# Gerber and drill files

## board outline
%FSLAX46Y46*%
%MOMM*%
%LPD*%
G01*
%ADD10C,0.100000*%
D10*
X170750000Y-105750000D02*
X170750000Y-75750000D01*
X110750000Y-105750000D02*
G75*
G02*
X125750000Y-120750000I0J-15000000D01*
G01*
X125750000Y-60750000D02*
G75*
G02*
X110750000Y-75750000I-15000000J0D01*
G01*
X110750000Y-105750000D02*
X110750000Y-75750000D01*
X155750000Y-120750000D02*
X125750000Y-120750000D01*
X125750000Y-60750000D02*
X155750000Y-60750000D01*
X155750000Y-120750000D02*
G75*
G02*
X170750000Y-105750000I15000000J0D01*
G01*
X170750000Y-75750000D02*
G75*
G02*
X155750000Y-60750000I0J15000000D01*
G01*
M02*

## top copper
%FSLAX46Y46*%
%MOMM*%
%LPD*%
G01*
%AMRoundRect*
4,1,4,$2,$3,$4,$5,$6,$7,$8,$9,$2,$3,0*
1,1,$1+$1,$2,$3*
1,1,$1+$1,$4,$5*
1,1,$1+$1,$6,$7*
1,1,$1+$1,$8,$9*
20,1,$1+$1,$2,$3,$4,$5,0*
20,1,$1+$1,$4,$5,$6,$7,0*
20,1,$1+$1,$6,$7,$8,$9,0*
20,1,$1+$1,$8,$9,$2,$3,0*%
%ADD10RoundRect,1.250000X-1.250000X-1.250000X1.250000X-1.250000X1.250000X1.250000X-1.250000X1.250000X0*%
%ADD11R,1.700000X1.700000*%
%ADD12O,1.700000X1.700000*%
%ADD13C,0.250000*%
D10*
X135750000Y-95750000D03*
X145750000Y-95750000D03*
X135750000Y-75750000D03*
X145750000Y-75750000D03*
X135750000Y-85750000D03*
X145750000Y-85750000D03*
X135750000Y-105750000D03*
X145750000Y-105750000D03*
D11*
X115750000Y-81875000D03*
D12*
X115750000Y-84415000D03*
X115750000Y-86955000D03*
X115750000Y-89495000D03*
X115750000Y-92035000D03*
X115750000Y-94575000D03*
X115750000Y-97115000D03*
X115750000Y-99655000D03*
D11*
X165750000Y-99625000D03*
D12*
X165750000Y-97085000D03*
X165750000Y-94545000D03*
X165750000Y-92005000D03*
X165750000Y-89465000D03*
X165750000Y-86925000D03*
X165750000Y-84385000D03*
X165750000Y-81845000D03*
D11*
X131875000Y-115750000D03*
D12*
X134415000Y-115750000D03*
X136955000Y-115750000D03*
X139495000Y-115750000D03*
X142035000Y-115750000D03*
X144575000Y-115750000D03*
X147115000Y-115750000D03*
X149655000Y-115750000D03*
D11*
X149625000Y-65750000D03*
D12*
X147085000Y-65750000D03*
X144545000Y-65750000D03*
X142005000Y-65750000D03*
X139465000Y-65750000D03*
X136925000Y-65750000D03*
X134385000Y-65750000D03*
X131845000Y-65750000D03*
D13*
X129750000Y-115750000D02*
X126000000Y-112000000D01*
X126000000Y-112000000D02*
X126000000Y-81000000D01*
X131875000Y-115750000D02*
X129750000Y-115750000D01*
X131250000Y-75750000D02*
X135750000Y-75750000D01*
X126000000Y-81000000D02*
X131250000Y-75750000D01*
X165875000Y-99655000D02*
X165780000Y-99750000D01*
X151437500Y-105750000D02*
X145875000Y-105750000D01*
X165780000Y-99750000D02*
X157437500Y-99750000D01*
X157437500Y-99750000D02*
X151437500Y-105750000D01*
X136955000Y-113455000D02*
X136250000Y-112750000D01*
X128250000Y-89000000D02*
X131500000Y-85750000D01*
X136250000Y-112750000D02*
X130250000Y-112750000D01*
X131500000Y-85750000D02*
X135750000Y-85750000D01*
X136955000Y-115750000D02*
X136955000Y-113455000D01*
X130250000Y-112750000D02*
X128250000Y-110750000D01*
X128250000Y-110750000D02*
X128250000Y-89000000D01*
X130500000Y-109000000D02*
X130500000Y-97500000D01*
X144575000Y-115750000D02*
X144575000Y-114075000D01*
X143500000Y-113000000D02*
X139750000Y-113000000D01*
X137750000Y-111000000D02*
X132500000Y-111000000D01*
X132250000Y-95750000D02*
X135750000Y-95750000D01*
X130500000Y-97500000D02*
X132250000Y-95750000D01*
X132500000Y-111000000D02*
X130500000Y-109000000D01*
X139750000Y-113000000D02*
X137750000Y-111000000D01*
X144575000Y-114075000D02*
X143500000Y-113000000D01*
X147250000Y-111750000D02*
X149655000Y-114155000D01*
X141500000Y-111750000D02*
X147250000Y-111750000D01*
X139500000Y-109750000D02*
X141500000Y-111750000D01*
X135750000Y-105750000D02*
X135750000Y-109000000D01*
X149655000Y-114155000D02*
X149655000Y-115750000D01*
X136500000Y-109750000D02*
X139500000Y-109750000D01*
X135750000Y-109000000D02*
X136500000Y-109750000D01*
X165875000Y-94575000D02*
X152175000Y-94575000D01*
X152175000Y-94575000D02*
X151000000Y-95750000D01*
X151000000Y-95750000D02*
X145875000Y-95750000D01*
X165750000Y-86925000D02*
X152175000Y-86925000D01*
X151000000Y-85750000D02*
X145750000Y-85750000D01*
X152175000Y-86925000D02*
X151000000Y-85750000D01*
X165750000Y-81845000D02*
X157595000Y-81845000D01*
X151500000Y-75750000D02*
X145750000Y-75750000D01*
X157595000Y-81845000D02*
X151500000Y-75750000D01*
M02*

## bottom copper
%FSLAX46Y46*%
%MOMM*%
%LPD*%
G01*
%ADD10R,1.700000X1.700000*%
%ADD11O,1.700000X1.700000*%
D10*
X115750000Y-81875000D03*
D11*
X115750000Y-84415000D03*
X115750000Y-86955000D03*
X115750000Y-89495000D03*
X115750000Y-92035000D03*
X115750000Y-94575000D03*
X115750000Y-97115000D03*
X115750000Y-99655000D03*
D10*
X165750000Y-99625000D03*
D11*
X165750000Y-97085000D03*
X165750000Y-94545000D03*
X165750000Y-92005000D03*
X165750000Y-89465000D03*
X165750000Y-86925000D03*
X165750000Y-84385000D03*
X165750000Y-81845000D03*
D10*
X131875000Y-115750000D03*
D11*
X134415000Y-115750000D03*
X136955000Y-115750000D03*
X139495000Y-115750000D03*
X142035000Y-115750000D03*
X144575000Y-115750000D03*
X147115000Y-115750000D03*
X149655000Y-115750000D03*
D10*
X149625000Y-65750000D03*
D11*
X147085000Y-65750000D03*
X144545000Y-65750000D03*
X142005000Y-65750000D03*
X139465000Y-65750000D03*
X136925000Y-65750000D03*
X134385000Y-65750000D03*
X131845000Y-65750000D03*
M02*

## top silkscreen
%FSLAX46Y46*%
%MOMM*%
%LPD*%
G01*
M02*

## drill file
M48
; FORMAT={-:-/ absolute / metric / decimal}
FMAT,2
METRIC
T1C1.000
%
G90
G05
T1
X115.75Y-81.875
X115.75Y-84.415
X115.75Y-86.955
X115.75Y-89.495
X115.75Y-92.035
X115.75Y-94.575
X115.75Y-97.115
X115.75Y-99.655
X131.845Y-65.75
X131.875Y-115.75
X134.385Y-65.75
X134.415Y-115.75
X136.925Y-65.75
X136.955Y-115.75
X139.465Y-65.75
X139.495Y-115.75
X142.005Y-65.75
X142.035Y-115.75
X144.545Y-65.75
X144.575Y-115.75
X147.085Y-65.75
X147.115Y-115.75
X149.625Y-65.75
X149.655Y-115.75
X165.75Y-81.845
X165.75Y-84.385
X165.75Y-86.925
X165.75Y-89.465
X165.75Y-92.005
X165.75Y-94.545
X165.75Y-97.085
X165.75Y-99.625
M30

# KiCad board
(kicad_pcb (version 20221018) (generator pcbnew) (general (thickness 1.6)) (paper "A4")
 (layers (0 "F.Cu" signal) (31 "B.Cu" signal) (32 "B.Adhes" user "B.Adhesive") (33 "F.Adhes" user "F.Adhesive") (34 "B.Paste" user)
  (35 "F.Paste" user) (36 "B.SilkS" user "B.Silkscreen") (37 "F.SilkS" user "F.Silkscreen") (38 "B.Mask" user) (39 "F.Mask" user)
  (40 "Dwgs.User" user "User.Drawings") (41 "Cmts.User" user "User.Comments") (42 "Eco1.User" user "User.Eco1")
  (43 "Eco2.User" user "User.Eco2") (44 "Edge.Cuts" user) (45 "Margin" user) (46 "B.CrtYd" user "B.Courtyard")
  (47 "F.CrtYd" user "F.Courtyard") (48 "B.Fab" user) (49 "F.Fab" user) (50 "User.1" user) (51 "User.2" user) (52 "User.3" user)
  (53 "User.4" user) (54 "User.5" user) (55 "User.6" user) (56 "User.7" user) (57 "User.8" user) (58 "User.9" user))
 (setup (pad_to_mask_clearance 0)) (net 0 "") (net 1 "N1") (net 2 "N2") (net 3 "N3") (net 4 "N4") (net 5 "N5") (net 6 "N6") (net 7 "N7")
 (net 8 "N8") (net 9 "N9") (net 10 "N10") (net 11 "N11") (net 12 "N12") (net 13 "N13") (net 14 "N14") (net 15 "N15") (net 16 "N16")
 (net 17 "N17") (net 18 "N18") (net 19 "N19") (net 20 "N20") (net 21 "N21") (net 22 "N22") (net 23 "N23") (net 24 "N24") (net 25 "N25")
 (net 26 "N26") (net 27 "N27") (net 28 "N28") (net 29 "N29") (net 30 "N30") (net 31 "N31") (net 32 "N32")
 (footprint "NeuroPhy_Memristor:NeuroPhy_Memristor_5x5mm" (layer "F.Cu") (at 140.75 95.75)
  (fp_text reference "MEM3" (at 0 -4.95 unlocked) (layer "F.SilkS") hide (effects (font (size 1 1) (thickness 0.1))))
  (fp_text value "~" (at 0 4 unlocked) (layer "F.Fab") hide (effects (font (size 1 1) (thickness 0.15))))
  (pad "1" smd roundrect (at -5 0) (size 5 5) (layers "F.Cu" "F.Mask") (roundrect_rratio 0.25) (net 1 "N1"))
  (pad "2" smd roundrect (at 5 0) (size 5 5) (layers "F.Cu" "F.Mask") (roundrect_rratio 0.25) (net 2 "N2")))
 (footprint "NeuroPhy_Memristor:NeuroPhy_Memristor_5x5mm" (layer "F.Cu") (at 140.75 75.75)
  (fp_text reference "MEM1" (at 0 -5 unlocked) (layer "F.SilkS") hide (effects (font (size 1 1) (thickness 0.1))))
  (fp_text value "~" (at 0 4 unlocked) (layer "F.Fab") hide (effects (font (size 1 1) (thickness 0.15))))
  (pad "1" smd roundrect (at -5 0) (size 5 5) (layers "F.Cu" "F.Mask") (roundrect_rratio 0.25) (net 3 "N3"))
  (pad "2" smd roundrect (at 5 0) (size 5 5) (layers "F.Cu" "F.Mask") (roundrect_rratio 0.25) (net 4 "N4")))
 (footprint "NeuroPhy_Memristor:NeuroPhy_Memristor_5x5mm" (layer "F.Cu") (at 140.75 85.75)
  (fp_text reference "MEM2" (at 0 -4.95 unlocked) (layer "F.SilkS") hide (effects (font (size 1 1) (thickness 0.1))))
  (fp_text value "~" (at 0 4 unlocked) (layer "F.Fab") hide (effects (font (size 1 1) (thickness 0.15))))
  (pad "1" smd roundrect (at -5 0) (size 5 5) (layers "F.Cu" "F.Mask") (roundrect_rratio 0.25) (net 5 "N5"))
  (pad "2" smd roundrect (at 5 0) (size 5 5) (layers "F.Cu" "F.Mask") (roundrect_rratio 0.25) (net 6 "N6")))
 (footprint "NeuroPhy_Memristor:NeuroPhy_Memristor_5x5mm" (layer "F.Cu") (at 140.75 105.75)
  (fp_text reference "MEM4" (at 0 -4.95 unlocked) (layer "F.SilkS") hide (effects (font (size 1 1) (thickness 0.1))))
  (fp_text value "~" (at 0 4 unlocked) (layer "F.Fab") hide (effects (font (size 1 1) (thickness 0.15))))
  (pad "1" smd roundrect (at -5 0) (size 5 5) (layers "F.Cu" "F.Mask") (roundrect_rratio 0.25) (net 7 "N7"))
  (pad "2" smd roundrect (at 5 0) (size 5 5) (layers "F.Cu" "F.Mask") (roundrect_rratio 0.25) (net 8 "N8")))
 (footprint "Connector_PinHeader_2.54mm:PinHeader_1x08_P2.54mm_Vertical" (layer "B.Cu") (at 115.75 81.875 180)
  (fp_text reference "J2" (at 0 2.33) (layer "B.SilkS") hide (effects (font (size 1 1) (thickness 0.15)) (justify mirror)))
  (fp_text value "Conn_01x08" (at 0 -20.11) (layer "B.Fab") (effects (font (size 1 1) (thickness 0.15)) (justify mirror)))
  (pad "1" thru_hole rect (at 0 0 180) (size 1.7 1.7) (drill 1) (layers "*.Cu" "*.Mask") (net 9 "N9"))
  (pad "2" thru_hole oval (at 0 -2.54 180) (size 1.7 1.7) (drill 1) (layers "*.Cu" "*.Mask") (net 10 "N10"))
  (pad "3" thru_hole oval (at 0 -5.08 180) (size 1.7 1.7) (drill 1) (layers "*.Cu" "*.Mask") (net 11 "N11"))
  (pad "4" thru_hole oval (at 0 -7.62 180) (size 1.7 1.7) (drill 1) (layers "*.Cu" "*.Mask") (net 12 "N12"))
  (pad "5" thru_hole oval (at 0 -10.16 180) (size 1.7 1.7) (drill 1) (layers "*.Cu" "*.Mask") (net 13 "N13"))
  (pad "6" thru_hole oval (at 0 -12.7 180) (size 1.7 1.7) (drill 1) (layers "*.Cu" "*.Mask") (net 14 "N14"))
  (pad "7" thru_hole oval (at 0 -15.24 180) (size 1.7 1.7) (drill 1) (layers "*.Cu" "*.Mask") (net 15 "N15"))
  (pad "8" thru_hole oval (at 0 -17.78 180) (size 1.7 1.7) (drill 1) (layers "*.Cu" "*.Mask") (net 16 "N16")))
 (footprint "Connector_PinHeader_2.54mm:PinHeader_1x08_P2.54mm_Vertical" (layer "B.Cu") (at 165.75 99.625)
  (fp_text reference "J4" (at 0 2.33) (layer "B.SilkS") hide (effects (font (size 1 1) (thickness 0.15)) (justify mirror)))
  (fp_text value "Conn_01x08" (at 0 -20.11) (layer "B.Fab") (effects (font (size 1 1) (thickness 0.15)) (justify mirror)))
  (pad "1" thru_hole rect (at 0 0) (size 1.7 1.7) (drill 1) (layers "*.Cu" "*.Mask") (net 8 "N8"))
  (pad "2" thru_hole oval (at 0 -2.54) (size 1.7 1.7) (drill 1) (layers "*.Cu" "*.Mask") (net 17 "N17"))
  (pad "3" thru_hole oval (at 0 -5.08) (size 1.7 1.7) (drill 1) (layers "*.Cu" "*.Mask") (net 2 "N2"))
  (pad "4" thru_hole oval (at 0 -7.62) (size 1.7 1.7) (drill 1) (layers "*.Cu" "*.Mask") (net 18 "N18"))
  (pad "5" thru_hole oval (at 0 -10.16) (size 1.7 1.7) (drill 1) (layers "*.Cu" "*.Mask") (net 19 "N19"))
  (pad "6" thru_hole oval (at 0 -12.7) (size 1.7 1.7) (drill 1) (layers "*.Cu" "*.Mask") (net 6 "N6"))
  (pad "7" thru_hole oval (at 0 -15.24) (size 1.7 1.7) (drill 1) (layers "*.Cu" "*.Mask") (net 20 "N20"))
  (pad "8" thru_hole oval (at 0 -17.78) (size 1.7 1.7) (drill 1) (layers "*.Cu" "*.Mask") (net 4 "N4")))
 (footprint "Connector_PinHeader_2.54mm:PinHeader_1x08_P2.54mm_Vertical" (layer "B.Cu") (at 131.875 115.75 -90)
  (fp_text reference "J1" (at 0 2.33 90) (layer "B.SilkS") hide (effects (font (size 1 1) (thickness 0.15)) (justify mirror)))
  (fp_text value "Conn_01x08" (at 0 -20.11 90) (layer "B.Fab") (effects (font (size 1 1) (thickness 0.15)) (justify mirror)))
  (pad "1" thru_hole rect (at 0 0 270) (size 1.7 1.7) (drill 1) (layers "*.Cu" "*.Mask") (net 3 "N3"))
  (pad "2" thru_hole oval (at 0 -2.54 270) (size 1.7 1.7) (drill 1) (layers "*.Cu" "*.Mask") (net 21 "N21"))
  (pad "3" thru_hole oval (at 0 -5.08 270) (size 1.7 1.7) (drill 1) (layers "*.Cu" "*.Mask") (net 5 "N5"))
  (pad "4" thru_hole oval (at 0 -7.62 270) (size 1.7 1.7) (drill 1) (layers "*.Cu" "*.Mask") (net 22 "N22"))
  (pad "5" thru_hole oval (at 0 -10.16 270) (size 1.7 1.7) (drill 1) (layers "*.Cu" "*.Mask") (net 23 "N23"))
  (pad "6" thru_hole oval (at 0 -12.7 270) (size 1.7 1.7) (drill 1) (layers "*.Cu" "*.Mask") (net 1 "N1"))
  (pad "7" thru_hole oval (at 0 -15.24 270) (size 1.7 1.7) (drill 1) (layers "*.Cu" "*.Mask") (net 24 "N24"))
  (pad "8" thru_hole oval (at 0 -17.78 270) (size 1.7 1.7) (drill 1) (layers "*.Cu" "*.Mask") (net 7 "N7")))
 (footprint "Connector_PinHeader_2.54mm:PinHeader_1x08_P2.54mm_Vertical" (layer "B.Cu") (at 149.625 65.75 90)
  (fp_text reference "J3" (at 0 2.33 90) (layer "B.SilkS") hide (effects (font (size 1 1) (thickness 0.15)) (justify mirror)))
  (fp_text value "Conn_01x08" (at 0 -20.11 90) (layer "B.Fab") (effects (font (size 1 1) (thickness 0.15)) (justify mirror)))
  (pad "1" thru_hole rect (at 0 0 90) (size 1.7 1.7) (drill 1) (layers "*.Cu" "*.Mask") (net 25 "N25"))
  (pad "2" thru_hole oval (at 0 -2.54 90) (size 1.7 1.7) (drill 1) (layers "*.Cu" "*.Mask") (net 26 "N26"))
  (pad "3" thru_hole oval (at 0 -5.08 90) (size 1.7 1.7) (drill 1) (layers "*.Cu" "*.Mask") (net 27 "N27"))
  (pad "4" thru_hole oval (at 0 -7.62 90) (size 1.7 1.7) (drill 1) (layers "*.Cu" "*.Mask") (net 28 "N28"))
  (pad "5" thru_hole oval (at 0 -10.16 90) (size 1.7 1.7) (drill 1) (layers "*.Cu" "*.Mask") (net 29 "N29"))
  (pad "6" thru_hole oval (at 0 -12.7 90) (size 1.7 1.7) (drill 1) (layers "*.Cu" "*.Mask") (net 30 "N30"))
  (pad "7" thru_hole oval (at 0 -15.24 90) (size 1.7 1.7) (drill 1) (layers "*.Cu" "*.Mask") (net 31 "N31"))
  (pad "8" thru_hole oval (at 0 -17.78 90) (size 1.7 1.7) (drill 1) (layers "*.Cu" "*.Mask") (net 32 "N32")))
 (gr_line (start 170.75 105.75) (end 170.75 75.75) (stroke (width 0.1) (type default)) (layer "Edge.Cuts"))
 (gr_arc (start 110.75 105.75) (mid 121.356602 110.143398) (end 125.75 120.75) (stroke (width 0.1) (type default)) (layer "Edge.Cuts"))
 (gr_arc (start 125.75 60.75) (mid 121.356602 71.356602) (end 110.75 75.75) (stroke (width 0.1) (type default)) (layer "Edge.Cuts"))
 (gr_line (start 110.75 105.75) (end 110.75 75.75) (stroke (width 0.1) (type default)) (layer "Edge.Cuts"))
 (gr_line (start 155.75 120.75) (end 125.75 120.75) (stroke (width 0.1) (type default)) (layer "Edge.Cuts"))
 (gr_line (start 125.75 60.75) (end 155.75 60.75) (stroke (width 0.1) (type default)) (layer "Edge.Cuts"))
 (gr_arc (start 155.75 120.75) (mid 160.143398 110.143398) (end 170.75 105.75) (stroke (width 0.1) (type default)) (layer "Edge.Cuts"))
 (gr_arc (start 170.75 75.75) (mid 160.143398 71.356602) (end 155.75 60.75) (stroke (width 0.1) (type default)) (layer "Edge.Cuts"))
 (segment (start 129.75 115.75) (end 126 112) (width 0.25) (layer "F.Cu") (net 3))
 (segment (start 126 112) (end 126 81) (width 0.25) (layer "F.Cu") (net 3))
 (segment (start 131.875 115.75) (end 129.75 115.75) (width 0.25) (layer "F.Cu") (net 3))
 (segment (start 131.25 75.75) (end 135.75 75.75) (width 0.25) (layer "F.Cu") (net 3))
 (segment (start 126 81) (end 131.25 75.75) (width 0.25) (layer "F.Cu") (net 3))
 (segment (start 165.875 99.655) (end 165.78 99.75) (width 0.25) (layer "F.Cu") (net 8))
 (segment (start 151.4375 105.75) (end 145.875 105.75) (width 0.25) (layer "F.Cu") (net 8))
 (segment (start 165.78 99.75) (end 157.4375 99.75) (width 0.25) (layer "F.Cu") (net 8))
 (segment (start 157.4375 99.75) (end 151.4375 105.75) (width 0.25) (layer "F.Cu") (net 8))
 (segment (start 136.955 113.455) (end 136.25 112.75) (width 0.25) (layer "F.Cu") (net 5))
 (segment (start 128.25 89) (end 131.5 85.75) (width 0.25) (layer "F.Cu") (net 5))
 (segment (start 136.25 112.75) (end 130.25 112.75) (width 0.25) (layer "F.Cu") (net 5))
 (segment (start 131.5 85.75) (end 135.75 85.75) (width 0.25) (layer "F.Cu") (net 5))
 (segment (start 136.955 115.75) (end 136.955 113.455) (width 0.25) (layer "F.Cu") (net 5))
 (segment (start 130.25 112.75) (end 128.25 110.75) (width 0.25) (layer "F.Cu") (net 5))
 (segment (start 128.25 110.75) (end 128.25 89) (width 0.25) (layer "F.Cu") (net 5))
 (segment (start 130.5 109) (end 130.5 97.5) (width 0.25) (layer "F.Cu") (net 1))
 (segment (start 144.575 115.75) (end 144.575 114.075) (width 0.25) (layer "F.Cu") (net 1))
 (segment (start 143.5 113) (end 139.75 113) (width 0.25) (layer "F.Cu") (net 1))
 (segment (start 137.75 111) (end 132.5 111) (width 0.25) (layer "F.Cu") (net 1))
 (segment (start 132.25 95.75) (end 135.75 95.75) (width 0.25) (layer "F.Cu") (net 1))
 (segment (start 130.5 97.5) (end 132.25 95.75) (width 0.25) (layer "F.Cu") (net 1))
 (segment (start 132.5 111) (end 130.5 109) (width 0.25) (layer "F.Cu") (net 1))
 (segment (start 139.75 113) (end 137.75 111) (width 0.25) (layer "F.Cu") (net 1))
 (segment (start 144.575 114.075) (end 143.5 113) (width 0.25) (layer "F.Cu") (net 1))
 (segment (start 147.25 111.75) (end 149.655 114.155) (width 0.25) (layer "F.Cu") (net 7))
 (segment (start 141.5 111.75) (end 147.25 111.75) (width 0.25) (layer "F.Cu") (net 7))
 (segment (start 139.5 109.75) (end 141.5 111.75) (width 0.25) (layer "F.Cu") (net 7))
 (segment (start 135.75 105.75) (end 135.75 109) (width 0.25) (layer "F.Cu") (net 7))
 (segment (start 149.655 114.155) (end 149.655 115.75) (width 0.25) (layer "F.Cu") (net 7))
 (segment (start 136.5 109.75) (end 139.5 109.75) (width 0.25) (layer "F.Cu") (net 7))
 (segment (start 135.75 109) (end 136.5 109.75) (width 0.25) (layer "F.Cu") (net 7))
 (segment (start 165.875 94.575) (end 152.175 94.575) (width 0.25) (layer "F.Cu") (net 2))
 (segment (start 152.175 94.575) (end 151 95.75) (width 0.25) (layer "F.Cu") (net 2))
 (segment (start 151 95.75) (end 145.875 95.75) (width 0.25) (layer "F.Cu") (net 2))
 (segment (start 165.75 86.925) (end 152.175 86.925) (width 0.25) (layer "F.Cu") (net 6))
 (segment (start 151 85.75) (end 145.75 85.75) (width 0.25) (layer "F.Cu") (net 6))
 (segment (start 152.175 86.925) (end 151 85.75) (width 0.25) (layer "F.Cu") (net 6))
 (segment (start 165.75 81.845) (end 157.595 81.845) (width 0.25) (layer "F.Cu") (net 4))
 (segment (start 151.5 75.75) (end 145.75 75.75) (width 0.25) (layer "F.Cu") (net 4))
 (segment (start 157.595 81.845) (end 151.5 75.75) (width 0.25) (layer "F.Cu") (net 4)))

